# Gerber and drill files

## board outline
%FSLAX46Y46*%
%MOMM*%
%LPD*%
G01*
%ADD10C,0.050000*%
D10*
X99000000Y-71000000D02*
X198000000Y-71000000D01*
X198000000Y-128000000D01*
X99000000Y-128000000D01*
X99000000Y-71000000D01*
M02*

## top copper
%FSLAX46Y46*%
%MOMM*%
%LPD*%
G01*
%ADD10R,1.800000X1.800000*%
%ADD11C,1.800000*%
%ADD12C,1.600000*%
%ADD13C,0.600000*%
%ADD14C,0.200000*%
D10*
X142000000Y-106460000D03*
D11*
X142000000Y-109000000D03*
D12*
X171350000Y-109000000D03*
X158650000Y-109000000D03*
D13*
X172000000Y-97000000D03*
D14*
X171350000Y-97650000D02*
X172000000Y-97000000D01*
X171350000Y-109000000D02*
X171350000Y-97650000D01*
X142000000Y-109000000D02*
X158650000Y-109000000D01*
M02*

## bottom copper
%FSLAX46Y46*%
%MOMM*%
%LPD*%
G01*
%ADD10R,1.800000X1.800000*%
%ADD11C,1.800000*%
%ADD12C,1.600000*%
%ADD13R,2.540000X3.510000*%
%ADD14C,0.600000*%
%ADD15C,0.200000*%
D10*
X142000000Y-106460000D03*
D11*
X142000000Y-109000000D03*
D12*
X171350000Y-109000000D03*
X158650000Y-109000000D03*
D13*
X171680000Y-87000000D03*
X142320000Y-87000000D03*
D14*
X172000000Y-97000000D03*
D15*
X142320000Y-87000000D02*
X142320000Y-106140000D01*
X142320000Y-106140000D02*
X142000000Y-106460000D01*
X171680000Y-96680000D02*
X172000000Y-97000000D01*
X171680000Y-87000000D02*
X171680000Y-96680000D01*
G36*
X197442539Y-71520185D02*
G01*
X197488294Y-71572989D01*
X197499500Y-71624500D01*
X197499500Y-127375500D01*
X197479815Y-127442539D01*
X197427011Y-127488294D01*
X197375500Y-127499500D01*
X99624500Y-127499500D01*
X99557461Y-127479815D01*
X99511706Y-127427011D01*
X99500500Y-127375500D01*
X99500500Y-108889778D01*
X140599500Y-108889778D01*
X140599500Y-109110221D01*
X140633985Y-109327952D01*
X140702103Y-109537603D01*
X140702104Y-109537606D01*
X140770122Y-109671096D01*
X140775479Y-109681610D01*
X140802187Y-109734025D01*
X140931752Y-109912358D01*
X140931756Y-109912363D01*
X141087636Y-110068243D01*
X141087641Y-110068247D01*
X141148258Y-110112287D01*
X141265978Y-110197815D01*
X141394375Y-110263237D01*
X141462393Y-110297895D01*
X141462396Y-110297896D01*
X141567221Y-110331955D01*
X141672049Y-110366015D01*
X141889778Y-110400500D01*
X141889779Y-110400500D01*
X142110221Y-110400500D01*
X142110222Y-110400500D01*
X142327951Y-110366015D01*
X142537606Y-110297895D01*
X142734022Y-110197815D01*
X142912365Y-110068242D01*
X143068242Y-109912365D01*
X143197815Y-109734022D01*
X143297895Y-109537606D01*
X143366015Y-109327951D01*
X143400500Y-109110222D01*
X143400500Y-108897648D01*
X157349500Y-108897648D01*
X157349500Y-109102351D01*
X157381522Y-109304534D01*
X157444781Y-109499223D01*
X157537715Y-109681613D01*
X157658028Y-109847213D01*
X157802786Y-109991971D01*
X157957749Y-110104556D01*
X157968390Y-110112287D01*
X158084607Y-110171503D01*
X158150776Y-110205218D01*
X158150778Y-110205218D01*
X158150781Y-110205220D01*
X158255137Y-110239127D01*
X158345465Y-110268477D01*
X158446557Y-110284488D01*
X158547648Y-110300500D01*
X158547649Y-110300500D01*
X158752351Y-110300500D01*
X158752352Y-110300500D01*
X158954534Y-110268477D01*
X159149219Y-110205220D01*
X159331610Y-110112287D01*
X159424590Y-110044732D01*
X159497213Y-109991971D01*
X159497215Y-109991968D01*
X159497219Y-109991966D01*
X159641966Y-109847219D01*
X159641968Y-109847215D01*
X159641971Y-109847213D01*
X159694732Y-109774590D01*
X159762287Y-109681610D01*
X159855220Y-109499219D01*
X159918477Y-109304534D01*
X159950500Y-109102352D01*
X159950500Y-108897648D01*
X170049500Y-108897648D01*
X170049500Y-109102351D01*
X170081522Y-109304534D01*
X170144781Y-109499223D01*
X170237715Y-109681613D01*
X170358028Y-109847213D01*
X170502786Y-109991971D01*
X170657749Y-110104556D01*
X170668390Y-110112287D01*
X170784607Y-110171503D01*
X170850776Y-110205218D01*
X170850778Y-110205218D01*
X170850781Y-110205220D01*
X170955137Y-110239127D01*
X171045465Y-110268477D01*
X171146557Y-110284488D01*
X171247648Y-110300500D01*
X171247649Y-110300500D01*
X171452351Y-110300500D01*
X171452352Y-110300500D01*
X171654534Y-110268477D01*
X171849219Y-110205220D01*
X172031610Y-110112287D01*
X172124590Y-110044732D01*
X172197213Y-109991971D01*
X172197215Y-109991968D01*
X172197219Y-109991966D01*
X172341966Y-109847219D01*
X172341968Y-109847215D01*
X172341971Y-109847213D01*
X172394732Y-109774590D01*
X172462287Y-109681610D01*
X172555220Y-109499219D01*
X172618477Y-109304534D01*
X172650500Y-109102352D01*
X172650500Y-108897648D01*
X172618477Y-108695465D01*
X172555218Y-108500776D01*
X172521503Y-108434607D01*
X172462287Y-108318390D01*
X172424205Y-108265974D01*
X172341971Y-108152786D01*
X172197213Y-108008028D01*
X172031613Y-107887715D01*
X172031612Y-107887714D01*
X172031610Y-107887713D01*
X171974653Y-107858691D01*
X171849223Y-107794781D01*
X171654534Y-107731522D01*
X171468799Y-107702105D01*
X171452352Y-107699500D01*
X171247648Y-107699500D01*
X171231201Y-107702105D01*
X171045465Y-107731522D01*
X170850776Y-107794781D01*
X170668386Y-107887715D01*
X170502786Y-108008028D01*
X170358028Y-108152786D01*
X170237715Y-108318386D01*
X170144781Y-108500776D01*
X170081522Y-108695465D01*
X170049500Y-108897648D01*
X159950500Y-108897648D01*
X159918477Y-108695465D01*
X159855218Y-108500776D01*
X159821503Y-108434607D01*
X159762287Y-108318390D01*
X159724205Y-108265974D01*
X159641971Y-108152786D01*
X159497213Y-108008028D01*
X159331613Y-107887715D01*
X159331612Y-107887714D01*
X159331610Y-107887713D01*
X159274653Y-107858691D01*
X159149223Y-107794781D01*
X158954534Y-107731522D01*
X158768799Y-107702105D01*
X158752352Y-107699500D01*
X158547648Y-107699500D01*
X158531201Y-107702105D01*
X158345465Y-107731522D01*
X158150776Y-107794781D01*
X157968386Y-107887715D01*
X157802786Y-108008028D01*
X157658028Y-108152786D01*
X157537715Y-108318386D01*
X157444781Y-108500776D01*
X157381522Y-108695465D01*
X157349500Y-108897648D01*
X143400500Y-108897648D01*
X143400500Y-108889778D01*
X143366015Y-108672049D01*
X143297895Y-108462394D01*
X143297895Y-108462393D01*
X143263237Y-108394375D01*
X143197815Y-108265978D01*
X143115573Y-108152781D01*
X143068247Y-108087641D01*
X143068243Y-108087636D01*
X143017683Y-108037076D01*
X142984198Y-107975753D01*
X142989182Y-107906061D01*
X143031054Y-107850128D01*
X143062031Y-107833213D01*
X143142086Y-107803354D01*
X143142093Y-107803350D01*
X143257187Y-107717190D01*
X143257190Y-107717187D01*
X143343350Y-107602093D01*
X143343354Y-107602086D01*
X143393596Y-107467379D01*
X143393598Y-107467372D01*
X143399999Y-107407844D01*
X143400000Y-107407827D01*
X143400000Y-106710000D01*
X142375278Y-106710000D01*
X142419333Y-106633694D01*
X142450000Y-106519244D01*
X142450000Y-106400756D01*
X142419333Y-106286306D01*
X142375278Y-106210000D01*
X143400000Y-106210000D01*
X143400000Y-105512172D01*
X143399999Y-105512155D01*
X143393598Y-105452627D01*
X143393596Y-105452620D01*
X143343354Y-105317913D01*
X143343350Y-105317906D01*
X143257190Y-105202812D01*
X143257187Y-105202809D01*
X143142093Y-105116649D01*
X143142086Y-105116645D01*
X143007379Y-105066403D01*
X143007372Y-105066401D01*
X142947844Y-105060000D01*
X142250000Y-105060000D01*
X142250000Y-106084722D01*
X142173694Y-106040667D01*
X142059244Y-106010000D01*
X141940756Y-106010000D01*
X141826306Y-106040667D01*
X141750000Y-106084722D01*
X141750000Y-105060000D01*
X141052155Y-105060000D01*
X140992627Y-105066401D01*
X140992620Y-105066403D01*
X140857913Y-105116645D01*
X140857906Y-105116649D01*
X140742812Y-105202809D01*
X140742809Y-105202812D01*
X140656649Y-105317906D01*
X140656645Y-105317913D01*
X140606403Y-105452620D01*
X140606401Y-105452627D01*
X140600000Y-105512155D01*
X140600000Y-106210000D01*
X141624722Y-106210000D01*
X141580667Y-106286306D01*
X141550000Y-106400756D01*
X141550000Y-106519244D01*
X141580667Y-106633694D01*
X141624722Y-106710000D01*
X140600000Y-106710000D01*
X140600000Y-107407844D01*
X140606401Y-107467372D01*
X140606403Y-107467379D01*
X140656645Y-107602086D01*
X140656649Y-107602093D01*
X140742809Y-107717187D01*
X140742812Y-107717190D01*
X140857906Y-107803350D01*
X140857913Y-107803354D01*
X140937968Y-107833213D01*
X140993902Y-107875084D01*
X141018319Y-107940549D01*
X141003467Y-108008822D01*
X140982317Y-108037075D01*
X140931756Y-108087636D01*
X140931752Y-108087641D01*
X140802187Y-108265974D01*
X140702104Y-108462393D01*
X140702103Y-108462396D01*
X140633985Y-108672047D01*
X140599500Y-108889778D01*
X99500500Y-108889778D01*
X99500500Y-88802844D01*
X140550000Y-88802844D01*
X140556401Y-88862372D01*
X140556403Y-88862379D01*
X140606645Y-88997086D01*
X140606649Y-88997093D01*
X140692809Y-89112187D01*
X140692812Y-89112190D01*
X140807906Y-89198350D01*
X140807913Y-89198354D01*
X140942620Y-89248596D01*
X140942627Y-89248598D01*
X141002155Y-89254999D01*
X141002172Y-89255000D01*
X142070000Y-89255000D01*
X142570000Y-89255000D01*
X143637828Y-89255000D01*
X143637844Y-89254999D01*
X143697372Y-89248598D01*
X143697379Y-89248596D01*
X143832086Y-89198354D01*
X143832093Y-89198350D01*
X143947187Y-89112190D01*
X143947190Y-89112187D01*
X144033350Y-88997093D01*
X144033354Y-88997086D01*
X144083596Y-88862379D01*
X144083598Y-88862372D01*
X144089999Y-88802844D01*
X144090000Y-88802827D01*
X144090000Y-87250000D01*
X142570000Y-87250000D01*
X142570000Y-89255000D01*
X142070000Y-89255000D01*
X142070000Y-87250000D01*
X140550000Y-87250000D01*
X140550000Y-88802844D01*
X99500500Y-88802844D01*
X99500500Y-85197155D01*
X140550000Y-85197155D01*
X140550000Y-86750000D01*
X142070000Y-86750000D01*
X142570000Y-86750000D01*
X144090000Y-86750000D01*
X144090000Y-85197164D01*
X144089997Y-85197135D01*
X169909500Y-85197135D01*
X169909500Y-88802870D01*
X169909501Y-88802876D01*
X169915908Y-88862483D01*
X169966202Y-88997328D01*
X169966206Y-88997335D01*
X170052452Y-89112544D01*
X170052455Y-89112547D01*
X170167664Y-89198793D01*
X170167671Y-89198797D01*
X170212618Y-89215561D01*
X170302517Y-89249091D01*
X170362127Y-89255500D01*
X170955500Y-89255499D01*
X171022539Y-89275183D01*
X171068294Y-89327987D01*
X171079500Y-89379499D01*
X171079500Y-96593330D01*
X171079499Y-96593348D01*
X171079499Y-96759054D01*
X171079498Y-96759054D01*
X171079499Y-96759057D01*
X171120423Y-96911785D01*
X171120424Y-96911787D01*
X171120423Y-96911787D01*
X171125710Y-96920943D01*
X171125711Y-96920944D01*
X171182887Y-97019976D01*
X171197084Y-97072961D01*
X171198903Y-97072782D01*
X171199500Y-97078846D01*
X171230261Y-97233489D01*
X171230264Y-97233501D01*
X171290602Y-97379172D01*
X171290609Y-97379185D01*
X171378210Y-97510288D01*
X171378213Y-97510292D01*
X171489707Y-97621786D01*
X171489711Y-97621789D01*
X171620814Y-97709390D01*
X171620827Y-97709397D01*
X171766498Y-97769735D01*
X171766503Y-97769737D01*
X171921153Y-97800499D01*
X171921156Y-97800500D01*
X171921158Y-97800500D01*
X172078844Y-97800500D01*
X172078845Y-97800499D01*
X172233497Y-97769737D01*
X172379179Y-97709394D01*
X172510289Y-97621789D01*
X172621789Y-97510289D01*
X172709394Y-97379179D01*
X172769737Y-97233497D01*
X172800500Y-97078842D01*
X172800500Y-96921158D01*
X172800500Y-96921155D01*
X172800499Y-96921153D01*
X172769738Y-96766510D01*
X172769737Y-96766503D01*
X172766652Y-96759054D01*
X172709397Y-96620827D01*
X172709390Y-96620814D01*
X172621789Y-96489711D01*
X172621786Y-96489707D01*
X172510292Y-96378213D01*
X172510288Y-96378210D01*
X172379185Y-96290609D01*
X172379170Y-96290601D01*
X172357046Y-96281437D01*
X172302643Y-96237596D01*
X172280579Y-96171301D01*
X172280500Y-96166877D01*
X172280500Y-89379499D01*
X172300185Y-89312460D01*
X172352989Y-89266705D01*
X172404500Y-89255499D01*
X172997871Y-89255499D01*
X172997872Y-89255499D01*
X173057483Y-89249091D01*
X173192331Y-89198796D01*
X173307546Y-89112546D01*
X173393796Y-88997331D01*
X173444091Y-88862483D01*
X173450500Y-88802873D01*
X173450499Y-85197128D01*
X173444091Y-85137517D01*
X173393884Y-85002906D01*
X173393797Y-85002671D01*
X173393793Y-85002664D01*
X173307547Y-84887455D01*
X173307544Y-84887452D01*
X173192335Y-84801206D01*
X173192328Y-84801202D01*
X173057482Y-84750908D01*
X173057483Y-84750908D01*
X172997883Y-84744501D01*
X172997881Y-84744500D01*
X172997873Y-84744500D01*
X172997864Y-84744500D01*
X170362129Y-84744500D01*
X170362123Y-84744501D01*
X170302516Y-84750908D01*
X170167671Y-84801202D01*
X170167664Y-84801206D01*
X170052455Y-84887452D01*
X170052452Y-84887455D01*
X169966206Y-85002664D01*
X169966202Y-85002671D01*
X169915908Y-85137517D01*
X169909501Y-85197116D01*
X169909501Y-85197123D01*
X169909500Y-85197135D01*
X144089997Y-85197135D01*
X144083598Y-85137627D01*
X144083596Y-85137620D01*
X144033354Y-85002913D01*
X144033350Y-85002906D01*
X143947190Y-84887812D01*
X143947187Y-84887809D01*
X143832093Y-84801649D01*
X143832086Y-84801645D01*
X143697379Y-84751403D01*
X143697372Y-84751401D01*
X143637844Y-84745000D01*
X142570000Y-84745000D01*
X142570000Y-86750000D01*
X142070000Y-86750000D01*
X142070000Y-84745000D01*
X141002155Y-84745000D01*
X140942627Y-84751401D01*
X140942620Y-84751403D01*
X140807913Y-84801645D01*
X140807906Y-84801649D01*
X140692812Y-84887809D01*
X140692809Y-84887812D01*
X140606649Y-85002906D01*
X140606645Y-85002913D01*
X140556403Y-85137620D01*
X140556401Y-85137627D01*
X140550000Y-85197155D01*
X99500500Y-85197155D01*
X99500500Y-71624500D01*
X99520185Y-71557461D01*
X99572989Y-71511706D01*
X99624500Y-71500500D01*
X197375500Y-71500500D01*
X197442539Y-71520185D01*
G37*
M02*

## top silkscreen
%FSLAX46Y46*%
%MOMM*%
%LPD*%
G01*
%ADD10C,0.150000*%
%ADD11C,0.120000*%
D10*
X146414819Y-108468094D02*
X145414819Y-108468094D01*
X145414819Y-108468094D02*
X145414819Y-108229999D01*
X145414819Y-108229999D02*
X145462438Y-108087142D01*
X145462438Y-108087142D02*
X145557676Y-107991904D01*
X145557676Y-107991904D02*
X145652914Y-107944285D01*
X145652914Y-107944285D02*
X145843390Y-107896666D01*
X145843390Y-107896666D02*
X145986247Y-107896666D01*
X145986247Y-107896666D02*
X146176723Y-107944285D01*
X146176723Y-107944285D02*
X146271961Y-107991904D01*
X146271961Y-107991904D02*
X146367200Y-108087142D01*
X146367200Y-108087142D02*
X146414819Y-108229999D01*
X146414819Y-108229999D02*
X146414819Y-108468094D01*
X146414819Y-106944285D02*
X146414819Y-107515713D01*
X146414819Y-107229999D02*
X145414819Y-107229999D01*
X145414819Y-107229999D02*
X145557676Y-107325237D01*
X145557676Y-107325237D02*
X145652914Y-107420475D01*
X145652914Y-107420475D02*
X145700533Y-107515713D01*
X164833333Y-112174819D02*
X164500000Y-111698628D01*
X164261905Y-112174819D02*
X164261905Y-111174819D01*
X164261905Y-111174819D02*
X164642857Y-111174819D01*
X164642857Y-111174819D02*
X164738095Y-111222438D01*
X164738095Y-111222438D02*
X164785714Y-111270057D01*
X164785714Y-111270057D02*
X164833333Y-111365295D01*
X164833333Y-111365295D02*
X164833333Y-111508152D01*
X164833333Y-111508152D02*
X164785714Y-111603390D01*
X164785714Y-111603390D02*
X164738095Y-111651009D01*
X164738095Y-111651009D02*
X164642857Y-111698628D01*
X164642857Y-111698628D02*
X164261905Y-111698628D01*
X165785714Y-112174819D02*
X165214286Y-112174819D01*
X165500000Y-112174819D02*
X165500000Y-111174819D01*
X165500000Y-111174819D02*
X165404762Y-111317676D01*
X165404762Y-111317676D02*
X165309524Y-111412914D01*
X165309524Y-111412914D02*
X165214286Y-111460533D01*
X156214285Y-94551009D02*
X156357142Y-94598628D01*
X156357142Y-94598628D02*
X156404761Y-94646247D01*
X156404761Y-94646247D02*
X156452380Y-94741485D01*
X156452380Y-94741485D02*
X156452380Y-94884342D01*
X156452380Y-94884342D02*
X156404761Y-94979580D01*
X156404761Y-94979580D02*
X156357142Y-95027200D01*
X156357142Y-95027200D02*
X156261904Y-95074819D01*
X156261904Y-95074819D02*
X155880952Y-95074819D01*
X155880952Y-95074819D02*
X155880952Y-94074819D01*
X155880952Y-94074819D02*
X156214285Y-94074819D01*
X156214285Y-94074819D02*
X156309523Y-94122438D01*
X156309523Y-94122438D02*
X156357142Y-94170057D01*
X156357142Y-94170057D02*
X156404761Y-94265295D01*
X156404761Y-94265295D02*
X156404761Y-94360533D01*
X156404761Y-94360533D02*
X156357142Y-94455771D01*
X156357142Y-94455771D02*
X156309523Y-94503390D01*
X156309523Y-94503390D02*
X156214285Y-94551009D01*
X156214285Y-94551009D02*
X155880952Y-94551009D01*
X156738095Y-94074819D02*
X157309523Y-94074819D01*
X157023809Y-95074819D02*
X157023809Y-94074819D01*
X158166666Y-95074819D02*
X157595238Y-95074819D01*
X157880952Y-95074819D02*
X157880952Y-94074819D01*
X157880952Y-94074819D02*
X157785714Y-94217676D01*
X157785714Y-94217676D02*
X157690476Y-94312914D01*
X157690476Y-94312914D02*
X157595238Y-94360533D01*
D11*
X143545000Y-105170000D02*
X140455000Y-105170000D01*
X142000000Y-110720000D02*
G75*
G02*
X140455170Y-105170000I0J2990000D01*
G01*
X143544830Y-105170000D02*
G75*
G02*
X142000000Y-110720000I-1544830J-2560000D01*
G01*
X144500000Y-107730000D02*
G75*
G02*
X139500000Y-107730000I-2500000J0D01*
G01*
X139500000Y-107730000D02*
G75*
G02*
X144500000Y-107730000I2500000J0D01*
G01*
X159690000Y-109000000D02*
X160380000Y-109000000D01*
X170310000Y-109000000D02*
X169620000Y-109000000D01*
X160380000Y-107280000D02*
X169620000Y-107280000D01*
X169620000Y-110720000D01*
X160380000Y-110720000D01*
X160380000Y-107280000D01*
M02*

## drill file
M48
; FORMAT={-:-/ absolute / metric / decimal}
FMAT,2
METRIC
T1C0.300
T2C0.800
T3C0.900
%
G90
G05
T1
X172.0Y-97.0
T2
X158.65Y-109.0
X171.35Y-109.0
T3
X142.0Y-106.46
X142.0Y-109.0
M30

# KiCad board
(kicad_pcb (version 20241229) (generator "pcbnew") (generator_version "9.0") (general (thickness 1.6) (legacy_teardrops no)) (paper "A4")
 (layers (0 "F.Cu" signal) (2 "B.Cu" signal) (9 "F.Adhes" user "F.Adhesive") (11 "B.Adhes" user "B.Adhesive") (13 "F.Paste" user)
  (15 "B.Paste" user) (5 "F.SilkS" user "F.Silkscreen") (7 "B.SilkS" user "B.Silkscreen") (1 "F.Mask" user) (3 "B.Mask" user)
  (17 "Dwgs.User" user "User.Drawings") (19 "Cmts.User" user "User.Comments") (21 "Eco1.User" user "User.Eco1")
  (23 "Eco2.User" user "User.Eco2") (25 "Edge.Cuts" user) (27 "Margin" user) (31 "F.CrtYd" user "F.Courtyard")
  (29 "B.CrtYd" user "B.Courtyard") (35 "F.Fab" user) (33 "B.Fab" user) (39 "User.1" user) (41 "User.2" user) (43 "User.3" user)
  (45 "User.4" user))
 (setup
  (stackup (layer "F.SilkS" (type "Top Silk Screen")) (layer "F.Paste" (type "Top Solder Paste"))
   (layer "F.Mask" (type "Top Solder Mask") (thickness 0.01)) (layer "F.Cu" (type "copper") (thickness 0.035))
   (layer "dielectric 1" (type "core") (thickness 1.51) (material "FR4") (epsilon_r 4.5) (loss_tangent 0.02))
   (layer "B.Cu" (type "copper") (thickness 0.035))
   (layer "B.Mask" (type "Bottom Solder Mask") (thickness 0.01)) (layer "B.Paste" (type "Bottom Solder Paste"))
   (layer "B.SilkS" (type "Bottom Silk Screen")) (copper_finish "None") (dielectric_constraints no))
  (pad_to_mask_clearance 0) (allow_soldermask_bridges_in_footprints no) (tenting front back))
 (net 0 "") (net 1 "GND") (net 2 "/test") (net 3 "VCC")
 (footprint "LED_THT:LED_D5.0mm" (layer "F.Cu") (at 142 106.46 -90)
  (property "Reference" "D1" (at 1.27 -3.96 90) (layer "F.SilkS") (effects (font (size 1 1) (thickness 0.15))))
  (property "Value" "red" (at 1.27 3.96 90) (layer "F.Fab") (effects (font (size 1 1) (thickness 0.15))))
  (fp_line (start -1.29 -1.545) (end -1.29 1.545) (stroke (width 0.12) (type solid)) (layer "F.SilkS"))
  (fp_arc (start 4.26 0) (mid 2.071779 2.880495) (end -1.29 1.54483) (stroke (width 0.12) (type solid)) (layer "F.SilkS"))
  (fp_arc (start -1.29 -1.54483) (mid 2.071779 -2.880495) (end 4.26 0) (stroke (width 0.12) (type solid)) (layer "F.SilkS"))
  (fp_circle (center 1.27 0) (end 3.77 0) (stroke (width 0.12) (type solid)) (fill no) (layer "F.SilkS"))
  (pad "1" thru_hole rect (at 0 0 270) (size 1.8 1.8) (drill 0.9) (layers "*.Cu" "*.Mask") (remove_unused_layers no) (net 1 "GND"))
  (pad "2" thru_hole circle (at 2.54 0 270) (size 1.8 1.8) (drill 0.9) (layers "*.Cu" "*.Mask") (remove_unused_layers no) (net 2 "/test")))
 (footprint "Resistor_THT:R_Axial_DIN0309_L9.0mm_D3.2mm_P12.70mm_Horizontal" (layer "F.Cu") (at 171.35 109 180)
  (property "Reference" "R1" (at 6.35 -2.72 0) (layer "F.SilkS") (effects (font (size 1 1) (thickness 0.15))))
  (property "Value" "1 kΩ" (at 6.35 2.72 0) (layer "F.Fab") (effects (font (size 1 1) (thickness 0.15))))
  (fp_line (start 11.66 0) (end 10.97 0) (stroke (width 0.12) (type solid)) (layer "F.SilkS"))
  (fp_line (start 1.04 0) (end 1.73 0) (stroke (width 0.12) (type solid)) (layer "F.SilkS"))
  (fp_rect (start 1.73 -1.72) (end 10.97 1.72) (stroke (width 0.12) (type solid)) (fill no) (layer "F.SilkS"))
  (pad "1" thru_hole circle (at 0 0 180) (size 1.6 1.6) (drill 0.8) (layers "*.Cu" "*.Mask") (remove_unused_layers no) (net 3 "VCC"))
  (pad "2" thru_hole circle (at 12.7 0 180) (size 1.6 1.6) (drill 0.8) (layers "*.Cu" "*.Mask") (remove_unused_layers no) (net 2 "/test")))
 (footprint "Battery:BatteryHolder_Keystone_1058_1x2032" (layer "B.Cu") (at 157 87 180)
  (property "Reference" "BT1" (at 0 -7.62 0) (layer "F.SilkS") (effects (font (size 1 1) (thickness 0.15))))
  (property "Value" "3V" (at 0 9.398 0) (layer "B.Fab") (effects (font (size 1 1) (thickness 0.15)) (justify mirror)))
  (pad "1" smd rect (at -14.68 0 180) (size 2.54 3.51) (layers "B.Cu" "B.Mask" "B.Paste") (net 3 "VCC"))
  (pad "2" smd rect (at 14.68 0 180) (size 2.54 3.51) (layers "B.Cu" "B.Mask" "B.Paste") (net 1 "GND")))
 (gr_rect (start 99 71) (end 198 128) (stroke (width 0.05) (type default)) (fill no) (layer "Edge.Cuts"))
 (segment (start 142.32 87) (end 142.32 106.14) (width 0.2) (layer "B.Cu") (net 1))
 (segment (start 142.32 106.14) (end 142 106.46) (width 0.2) (layer "B.Cu") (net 1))
 (segment (start 171.35 97.65) (end 172 97) (width 0.2) (layer "F.Cu") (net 3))
 (segment (start 171.35 109) (end 171.35 97.65) (width 0.2) (layer "F.Cu") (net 3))
 (via (at 172 97) (size 0.6) (drill 0.3) (layers "F.Cu" "B.Cu") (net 3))
 (segment (start 171.68 96.68) (end 172 97) (width 0.2) (layer "B.Cu") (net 3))
 (segment (start 171.68 87) (end 171.68 96.68) (width 0.2) (layer "B.Cu") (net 3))
 (segment (start 142 109) (end 158.65 109) (width 0.2) (layer "F.Cu") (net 2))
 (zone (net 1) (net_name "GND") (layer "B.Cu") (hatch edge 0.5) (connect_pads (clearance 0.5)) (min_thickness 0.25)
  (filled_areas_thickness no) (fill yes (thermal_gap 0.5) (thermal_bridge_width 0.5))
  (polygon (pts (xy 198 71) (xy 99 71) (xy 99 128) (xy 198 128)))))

